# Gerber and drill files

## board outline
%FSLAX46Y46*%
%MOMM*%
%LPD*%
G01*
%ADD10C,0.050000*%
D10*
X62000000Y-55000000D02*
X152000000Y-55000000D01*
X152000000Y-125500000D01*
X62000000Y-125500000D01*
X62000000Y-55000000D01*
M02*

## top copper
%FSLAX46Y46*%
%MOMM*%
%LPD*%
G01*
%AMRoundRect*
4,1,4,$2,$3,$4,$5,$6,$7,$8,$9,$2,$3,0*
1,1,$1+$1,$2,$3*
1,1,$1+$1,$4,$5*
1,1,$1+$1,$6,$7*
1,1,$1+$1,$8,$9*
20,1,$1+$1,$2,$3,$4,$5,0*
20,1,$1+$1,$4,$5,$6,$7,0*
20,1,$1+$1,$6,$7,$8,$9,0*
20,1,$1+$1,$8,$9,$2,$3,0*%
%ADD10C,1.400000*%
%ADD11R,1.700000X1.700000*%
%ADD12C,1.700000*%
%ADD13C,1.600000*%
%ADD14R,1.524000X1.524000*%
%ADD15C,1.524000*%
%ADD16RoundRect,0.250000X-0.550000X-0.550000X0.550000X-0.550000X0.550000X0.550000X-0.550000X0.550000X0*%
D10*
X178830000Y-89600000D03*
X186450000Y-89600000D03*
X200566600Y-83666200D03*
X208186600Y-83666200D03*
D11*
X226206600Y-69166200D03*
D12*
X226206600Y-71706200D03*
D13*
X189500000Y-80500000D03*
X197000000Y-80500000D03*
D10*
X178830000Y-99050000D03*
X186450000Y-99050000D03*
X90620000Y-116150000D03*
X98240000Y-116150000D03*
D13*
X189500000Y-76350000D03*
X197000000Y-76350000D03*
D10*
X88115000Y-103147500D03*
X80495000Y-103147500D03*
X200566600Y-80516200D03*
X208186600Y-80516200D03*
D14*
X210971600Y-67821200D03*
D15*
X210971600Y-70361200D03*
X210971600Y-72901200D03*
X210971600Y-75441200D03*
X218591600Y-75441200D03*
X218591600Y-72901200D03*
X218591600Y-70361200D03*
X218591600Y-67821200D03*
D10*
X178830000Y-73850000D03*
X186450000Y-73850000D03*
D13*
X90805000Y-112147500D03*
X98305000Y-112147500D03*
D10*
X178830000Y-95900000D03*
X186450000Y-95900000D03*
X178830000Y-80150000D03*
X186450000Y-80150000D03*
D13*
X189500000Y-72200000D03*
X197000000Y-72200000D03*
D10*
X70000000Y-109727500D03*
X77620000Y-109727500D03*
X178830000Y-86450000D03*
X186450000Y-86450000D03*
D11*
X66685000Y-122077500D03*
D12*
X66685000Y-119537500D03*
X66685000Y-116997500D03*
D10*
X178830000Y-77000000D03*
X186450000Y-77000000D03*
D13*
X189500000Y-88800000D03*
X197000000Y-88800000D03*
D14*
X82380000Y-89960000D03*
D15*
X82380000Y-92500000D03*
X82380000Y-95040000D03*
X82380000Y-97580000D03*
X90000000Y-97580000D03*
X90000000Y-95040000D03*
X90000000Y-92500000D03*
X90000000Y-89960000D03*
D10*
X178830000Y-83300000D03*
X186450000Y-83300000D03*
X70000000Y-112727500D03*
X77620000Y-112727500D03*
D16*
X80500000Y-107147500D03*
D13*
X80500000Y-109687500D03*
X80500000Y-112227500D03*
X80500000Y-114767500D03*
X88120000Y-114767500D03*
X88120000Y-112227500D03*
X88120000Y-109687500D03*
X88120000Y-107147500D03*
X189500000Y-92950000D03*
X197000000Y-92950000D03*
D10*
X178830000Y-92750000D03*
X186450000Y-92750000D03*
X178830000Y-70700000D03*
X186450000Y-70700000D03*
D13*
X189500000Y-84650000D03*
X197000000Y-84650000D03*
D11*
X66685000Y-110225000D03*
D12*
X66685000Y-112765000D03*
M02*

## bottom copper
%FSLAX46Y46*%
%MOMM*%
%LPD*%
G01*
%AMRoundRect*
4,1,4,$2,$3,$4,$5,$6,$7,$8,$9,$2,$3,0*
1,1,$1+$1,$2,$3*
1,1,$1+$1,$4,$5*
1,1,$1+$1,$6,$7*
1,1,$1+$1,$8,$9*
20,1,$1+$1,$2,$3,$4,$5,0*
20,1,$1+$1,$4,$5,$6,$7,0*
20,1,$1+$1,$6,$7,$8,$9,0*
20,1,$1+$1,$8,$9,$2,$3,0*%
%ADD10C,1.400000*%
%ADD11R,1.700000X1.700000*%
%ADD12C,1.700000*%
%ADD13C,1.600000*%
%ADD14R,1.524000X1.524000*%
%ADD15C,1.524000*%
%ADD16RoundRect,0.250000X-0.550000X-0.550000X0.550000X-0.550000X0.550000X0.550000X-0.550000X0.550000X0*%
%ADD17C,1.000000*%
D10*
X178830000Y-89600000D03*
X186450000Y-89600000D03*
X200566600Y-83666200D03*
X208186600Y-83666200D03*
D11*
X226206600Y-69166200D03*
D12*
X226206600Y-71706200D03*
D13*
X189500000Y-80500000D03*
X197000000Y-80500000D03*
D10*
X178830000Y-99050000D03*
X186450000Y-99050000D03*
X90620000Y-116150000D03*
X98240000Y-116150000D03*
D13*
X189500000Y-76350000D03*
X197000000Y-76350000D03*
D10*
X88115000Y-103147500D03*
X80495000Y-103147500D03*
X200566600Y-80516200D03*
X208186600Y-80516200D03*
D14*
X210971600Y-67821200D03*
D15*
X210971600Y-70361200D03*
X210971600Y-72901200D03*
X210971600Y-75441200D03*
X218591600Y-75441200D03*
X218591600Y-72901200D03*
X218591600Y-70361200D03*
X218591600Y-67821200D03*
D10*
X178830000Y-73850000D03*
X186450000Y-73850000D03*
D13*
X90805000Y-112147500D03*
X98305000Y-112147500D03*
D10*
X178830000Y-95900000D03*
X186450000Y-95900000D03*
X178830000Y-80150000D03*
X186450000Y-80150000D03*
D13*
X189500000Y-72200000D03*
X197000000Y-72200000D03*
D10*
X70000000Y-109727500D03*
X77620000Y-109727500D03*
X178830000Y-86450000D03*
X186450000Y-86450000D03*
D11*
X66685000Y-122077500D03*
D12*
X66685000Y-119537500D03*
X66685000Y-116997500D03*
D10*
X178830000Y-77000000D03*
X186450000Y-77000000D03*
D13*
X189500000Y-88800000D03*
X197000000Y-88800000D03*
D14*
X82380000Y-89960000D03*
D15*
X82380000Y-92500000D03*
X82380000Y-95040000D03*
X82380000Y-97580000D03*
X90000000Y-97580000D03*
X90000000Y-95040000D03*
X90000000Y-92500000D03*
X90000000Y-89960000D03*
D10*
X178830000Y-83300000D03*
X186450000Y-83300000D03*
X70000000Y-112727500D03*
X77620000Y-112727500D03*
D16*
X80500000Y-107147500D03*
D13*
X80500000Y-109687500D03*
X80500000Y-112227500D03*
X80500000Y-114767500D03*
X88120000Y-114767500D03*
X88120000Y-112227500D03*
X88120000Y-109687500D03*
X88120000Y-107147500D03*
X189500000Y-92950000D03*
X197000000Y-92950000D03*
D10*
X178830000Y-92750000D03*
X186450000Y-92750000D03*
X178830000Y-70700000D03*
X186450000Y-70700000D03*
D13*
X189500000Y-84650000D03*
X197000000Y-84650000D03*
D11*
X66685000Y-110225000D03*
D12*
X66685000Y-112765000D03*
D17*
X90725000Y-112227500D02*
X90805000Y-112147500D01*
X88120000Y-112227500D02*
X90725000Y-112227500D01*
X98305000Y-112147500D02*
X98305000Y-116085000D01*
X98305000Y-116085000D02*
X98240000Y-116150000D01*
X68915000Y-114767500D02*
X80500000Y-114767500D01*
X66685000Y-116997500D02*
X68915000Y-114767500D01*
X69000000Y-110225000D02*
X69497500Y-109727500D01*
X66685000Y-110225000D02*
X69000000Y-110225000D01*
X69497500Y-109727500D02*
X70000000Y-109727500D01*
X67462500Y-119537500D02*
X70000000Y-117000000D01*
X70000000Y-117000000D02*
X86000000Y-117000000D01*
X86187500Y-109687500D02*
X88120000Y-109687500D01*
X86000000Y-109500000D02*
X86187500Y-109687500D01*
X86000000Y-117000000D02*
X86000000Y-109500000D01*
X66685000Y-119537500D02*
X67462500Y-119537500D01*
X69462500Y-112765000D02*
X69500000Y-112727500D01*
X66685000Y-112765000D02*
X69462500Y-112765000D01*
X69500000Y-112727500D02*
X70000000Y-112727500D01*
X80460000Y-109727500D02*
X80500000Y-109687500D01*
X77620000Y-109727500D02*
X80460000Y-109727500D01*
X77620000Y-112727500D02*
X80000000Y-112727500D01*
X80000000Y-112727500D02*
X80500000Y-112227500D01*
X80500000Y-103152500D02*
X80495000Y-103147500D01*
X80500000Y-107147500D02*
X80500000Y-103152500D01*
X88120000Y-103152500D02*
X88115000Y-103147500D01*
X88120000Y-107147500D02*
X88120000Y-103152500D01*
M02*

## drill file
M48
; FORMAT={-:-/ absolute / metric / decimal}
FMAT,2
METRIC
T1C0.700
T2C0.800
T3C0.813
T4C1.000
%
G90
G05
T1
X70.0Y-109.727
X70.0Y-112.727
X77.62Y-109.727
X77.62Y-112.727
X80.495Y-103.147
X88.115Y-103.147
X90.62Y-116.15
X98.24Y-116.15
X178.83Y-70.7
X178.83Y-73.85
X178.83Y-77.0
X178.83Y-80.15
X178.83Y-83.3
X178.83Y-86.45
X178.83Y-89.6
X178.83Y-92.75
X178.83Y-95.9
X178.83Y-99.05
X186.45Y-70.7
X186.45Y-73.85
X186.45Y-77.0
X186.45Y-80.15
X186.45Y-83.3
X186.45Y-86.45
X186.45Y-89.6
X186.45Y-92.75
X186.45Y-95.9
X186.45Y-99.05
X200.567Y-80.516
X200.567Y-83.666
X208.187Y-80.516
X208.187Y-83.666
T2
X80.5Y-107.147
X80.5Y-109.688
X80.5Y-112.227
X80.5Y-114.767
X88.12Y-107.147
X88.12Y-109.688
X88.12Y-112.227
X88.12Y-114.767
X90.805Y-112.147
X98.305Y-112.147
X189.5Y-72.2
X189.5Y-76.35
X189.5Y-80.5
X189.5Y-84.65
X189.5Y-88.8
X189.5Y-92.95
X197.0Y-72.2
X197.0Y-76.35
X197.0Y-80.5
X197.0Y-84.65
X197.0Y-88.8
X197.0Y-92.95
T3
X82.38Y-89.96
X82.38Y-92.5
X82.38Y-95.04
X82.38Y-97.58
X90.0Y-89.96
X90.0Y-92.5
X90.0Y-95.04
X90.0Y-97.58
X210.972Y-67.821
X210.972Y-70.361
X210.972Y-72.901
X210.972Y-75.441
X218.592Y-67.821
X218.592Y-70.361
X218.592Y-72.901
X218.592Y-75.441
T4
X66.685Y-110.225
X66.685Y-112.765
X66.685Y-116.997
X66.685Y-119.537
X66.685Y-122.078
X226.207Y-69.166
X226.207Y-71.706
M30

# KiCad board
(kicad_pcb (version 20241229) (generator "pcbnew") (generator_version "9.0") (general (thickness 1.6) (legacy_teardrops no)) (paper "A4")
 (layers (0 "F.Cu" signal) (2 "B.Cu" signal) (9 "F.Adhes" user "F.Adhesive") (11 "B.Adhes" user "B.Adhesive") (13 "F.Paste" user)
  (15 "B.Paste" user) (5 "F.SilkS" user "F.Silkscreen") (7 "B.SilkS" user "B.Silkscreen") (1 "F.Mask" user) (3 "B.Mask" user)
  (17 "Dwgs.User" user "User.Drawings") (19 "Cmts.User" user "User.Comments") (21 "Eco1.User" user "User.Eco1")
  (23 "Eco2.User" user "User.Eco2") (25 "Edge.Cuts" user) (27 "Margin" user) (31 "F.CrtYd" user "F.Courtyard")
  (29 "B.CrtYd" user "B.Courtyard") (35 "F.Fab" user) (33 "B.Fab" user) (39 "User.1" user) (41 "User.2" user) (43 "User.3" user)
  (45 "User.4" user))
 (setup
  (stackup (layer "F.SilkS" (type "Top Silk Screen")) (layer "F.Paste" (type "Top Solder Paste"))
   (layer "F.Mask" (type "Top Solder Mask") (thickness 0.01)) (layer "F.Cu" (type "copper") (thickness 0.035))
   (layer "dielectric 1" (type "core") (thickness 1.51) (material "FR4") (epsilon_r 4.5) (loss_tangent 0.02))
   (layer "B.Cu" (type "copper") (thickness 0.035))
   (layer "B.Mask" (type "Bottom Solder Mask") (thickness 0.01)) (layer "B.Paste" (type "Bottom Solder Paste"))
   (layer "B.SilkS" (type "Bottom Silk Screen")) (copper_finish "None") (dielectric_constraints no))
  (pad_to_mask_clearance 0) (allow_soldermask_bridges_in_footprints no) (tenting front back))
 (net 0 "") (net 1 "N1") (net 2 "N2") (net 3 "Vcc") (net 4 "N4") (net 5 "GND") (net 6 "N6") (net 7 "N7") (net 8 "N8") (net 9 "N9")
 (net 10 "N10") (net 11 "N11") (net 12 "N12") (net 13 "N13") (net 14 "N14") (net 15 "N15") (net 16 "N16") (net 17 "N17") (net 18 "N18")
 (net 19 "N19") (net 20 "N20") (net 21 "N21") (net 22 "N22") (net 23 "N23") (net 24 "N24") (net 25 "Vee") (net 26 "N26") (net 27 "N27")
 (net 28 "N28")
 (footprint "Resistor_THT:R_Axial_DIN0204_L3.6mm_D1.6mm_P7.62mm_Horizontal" (layer "F.Cu") (at 178.83 89.6)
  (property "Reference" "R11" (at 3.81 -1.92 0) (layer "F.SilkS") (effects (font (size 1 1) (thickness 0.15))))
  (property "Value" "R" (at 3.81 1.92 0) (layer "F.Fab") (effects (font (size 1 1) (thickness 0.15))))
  (pad "1" thru_hole circle (at 0 0) (size 1.4 1.4) (drill 0.7) (layers "*.Cu" "*.Mask") (remove_unused_layers no) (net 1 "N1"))
  (pad "2" thru_hole circle (at 7.62 0) (size 1.4 1.4) (drill 0.7) (layers "*.Cu" "*.Mask") (remove_unused_layers no) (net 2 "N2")))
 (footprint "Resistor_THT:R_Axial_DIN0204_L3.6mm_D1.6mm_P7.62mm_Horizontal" (layer "F.Cu") (at 200.5666 83.6662)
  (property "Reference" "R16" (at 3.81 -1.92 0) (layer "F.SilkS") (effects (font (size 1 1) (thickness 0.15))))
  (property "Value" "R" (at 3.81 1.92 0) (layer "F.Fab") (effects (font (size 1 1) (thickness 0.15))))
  (pad "1" thru_hole circle (at 0 0) (size 1.4 1.4) (drill 0.7) (layers "*.Cu" "*.Mask") (remove_unused_layers no) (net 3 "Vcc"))
  (pad "2" thru_hole circle (at 7.62 0) (size 1.4 1.4) (drill 0.7) (layers "*.Cu" "*.Mask") (remove_unused_layers no) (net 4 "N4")))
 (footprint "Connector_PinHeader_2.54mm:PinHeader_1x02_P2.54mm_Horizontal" (layer "F.Cu") (at 226.2066 69.1662)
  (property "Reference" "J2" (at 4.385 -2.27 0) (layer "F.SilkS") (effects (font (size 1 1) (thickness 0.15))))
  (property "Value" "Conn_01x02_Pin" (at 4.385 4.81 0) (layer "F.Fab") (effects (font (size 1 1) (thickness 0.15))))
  (pad "1" thru_hole rect (at 0 0) (size 1.7 1.7) (drill 1) (layers "*.Cu" "*.Mask") (remove_unused_layers no) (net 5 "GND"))
  (pad "2" thru_hole circle (at 0 2.54) (size 1.7 1.7) (drill 1) (layers "*.Cu" "*.Mask") (remove_unused_layers no) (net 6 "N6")))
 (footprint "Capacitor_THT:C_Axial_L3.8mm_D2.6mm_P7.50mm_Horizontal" (layer "F.Cu") (at 189.5 80.5)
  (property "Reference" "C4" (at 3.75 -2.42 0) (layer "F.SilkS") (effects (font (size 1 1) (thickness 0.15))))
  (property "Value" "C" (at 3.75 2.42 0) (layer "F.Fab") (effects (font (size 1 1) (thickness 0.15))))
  (pad "1" thru_hole circle (at 0 0) (size 1.6 1.6) (drill 0.8) (layers "*.Cu" "*.Mask") (remove_unused_layers no) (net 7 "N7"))
  (pad "2" thru_hole circle (at 7.5 0) (size 1.6 1.6) (drill 0.8) (layers "*.Cu" "*.Mask") (remove_unused_layers no) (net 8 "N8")))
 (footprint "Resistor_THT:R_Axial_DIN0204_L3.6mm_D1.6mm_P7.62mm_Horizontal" (layer "F.Cu") (at 178.83 99.05)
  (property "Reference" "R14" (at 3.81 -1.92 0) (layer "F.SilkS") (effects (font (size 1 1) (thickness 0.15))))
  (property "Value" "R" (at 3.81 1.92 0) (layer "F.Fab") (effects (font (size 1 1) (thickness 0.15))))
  (pad "1" thru_hole circle (at 0 0) (size 1.4 1.4) (drill 0.7) (layers "*.Cu" "*.Mask") (remove_unused_layers no) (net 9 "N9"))
  (pad "2" thru_hole circle (at 7.62 0) (size 1.4 1.4) (drill 0.7) (layers "*.Cu" "*.Mask") (remove_unused_layers no) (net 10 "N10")))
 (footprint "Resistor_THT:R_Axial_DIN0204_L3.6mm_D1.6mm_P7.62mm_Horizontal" (layer "F.Cu") (at 90.62 116.15)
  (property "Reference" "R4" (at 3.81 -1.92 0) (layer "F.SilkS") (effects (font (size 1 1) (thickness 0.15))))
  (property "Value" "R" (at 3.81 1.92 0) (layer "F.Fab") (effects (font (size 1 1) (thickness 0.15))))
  (pad "1" thru_hole circle (at 0 0) (size 1.4 1.4) (drill 0.7) (layers "*.Cu" "*.Mask") (remove_unused_layers no) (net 5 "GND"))
  (pad "2" thru_hole circle (at 7.62 0) (size 1.4 1.4) (drill 0.7) (layers "*.Cu" "*.Mask") (remove_unused_layers no) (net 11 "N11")))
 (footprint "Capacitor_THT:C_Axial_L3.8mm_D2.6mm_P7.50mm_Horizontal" (layer "F.Cu") (at 189.5 76.35)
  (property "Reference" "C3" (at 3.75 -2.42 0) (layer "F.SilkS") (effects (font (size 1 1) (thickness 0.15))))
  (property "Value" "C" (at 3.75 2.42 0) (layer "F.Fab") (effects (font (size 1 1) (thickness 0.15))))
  (pad "1" thru_hole circle (at 0 0) (size 1.6 1.6) (drill 0.8) (layers "*.Cu" "*.Mask") (remove_unused_layers no) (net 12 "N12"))
  (pad "2" thru_hole circle (at 7.5 0) (size 1.6 1.6) (drill 0.8) (layers "*.Cu" "*.Mask") (remove_unused_layers no) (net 5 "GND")))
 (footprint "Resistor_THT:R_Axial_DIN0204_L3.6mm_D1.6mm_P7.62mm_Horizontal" (layer "F.Cu") (at 88.115 103.1475 180)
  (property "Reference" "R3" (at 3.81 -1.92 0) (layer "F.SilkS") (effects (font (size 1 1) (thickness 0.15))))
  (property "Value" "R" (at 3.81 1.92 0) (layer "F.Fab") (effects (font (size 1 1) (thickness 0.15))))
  (pad "1" thru_hole circle (at 0 0 180) (size 1.4 1.4) (drill 0.7) (layers "*.Cu" "*.Mask") (remove_unused_layers no) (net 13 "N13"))
  (pad "2" thru_hole circle (at 7.62 0 180) (size 1.4 1.4) (drill 0.7) (layers "*.Cu" "*.Mask") (remove_unused_layers no) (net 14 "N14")))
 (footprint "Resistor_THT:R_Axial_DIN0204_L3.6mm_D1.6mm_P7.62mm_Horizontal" (layer "F.Cu") (at 200.5666 80.5162)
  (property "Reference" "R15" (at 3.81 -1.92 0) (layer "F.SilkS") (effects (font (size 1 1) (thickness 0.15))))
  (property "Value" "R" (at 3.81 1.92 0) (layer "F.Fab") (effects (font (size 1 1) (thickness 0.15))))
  (pad "1" thru_hole circle (at 0 0) (size 1.4 1.4) (drill 0.7) (layers "*.Cu" "*.Mask") (remove_unused_layers no) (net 5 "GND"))
  (pad "2" thru_hole circle (at 7.62 0) (size 1.4 1.4) (drill 0.7) (layers "*.Cu" "*.Mask") (remove_unused_layers no) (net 4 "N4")))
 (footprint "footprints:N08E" (layer "F.Cu") (at 218.5916 75.4412)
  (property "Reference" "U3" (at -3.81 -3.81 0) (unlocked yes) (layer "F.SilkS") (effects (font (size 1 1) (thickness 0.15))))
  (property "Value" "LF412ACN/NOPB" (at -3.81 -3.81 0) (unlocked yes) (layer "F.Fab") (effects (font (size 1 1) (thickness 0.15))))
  (pad "1" thru_hole rect (at -7.62 -7.62) (size 1.524 1.524) (drill 0.8128) (layers "*.Cu" "*.Mask") (remove_unused_layers no)
   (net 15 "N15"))
  (pad "2" thru_hole circle (at -7.62 -5.08) (size 1.524 1.524) (drill 0.8128) (layers "*.Cu" "*.Mask") (remove_unused_layers no)
   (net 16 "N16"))
  (pad "3" thru_hole circle (at -7.62 -2.54) (size 1.524 1.524) (drill 0.8128) (layers "*.Cu" "*.Mask") (remove_unused_layers no)
   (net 5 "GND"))
  (pad "4" thru_hole circle (at -7.62 0) (size 1.524 1.524) (drill 0.8128) (layers "*.Cu" "*.Mask") (remove_unused_layers no))
  (pad "5" thru_hole circle (at 0 0) (size 1.524 1.524) (drill 0.8128) (layers "*.Cu" "*.Mask") (remove_unused_layers no) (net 4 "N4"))
  (pad "6" thru_hole circle (at 0 -2.54) (size 1.524 1.524) (drill 0.8128) (layers "*.Cu" "*.Mask") (remove_unused_layers no) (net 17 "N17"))
  (pad "7" thru_hole circle (at 0 -5.08) (size 1.524 1.524) (drill 0.8128) (layers "*.Cu" "*.Mask") (remove_unused_layers no) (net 6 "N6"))
  (pad "8" thru_hole circle (at 0 -7.62) (size 1.524 1.524) (drill 0.8128) (layers "*.Cu" "*.Mask") (remove_unused_layers no)))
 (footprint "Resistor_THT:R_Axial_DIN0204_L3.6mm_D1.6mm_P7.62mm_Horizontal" (layer "F.Cu") (at 178.83 73.85)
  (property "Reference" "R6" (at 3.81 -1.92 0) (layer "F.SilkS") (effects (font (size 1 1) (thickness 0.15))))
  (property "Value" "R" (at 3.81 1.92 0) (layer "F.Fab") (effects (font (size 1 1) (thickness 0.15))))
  (pad "1" thru_hole circle (at 0 0) (size 1.4 1.4) (drill 0.7) (layers "*.Cu" "*.Mask") (remove_unused_layers no) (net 12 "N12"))
  (pad "2" thru_hole circle (at 7.62 0) (size 1.4 1.4) (drill 0.7) (layers "*.Cu" "*.Mask") (remove_unused_layers no) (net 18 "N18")))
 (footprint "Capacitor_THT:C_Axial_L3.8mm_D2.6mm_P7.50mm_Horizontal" (layer "F.Cu") (at 90.805 112.1475)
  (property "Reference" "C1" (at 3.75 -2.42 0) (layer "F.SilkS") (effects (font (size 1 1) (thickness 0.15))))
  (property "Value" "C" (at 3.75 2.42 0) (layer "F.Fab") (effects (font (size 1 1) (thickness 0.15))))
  (pad "1" thru_hole circle (at 0 0) (size 1.6 1.6) (drill 0.8) (layers "*.Cu" "*.Mask") (remove_unused_layers no) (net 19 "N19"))
  (pad "2" thru_hole circle (at 7.5 0) (size 1.6 1.6) (drill 0.8) (layers "*.Cu" "*.Mask") (remove_unused_layers no) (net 11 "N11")))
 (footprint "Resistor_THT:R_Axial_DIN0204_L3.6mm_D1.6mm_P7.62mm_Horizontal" (layer "F.Cu") (at 178.83 95.9)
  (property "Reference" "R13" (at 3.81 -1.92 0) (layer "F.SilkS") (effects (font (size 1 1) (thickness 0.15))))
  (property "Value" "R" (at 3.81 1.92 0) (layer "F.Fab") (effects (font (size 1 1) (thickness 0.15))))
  (pad "1" thru_hole circle (at 0 0) (size 1.4 1.4) (drill 0.7) (layers "*.Cu" "*.Mask") (remove_unused_layers no) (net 5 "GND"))
  (pad "2" thru_hole circle (at 7.62 0) (size 1.4 1.4) (drill 0.7) (layers "*.Cu" "*.Mask") (remove_unused_layers no) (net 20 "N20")))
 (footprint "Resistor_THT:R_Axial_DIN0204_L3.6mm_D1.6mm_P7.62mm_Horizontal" (layer "F.Cu") (at 178.83 80.15)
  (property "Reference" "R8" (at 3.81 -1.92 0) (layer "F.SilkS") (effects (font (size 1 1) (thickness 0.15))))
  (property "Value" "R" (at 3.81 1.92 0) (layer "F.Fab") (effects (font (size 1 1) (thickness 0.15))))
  (pad "1" thru_hole circle (at 0 0) (size 1.4 1.4) (drill 0.7) (layers "*.Cu" "*.Mask") (remove_unused_layers no) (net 5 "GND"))
  (pad "2" thru_hole circle (at 7.62 0) (size 1.4 1.4) (drill 0.7) (layers "*.Cu" "*.Mask") (remove_unused_layers no) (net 7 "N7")))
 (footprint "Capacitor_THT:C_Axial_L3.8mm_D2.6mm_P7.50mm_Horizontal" (layer "F.Cu") (at 189.5 72.2)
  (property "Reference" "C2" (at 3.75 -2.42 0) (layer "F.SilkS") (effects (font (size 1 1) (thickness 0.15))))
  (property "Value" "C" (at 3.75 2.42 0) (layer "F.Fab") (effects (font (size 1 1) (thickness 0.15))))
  (pad "1" thru_hole circle (at 0 0) (size 1.6 1.6) (drill 0.8) (layers "*.Cu" "*.Mask") (remove_unused_layers no) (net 12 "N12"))
  (pad "2" thru_hole circle (at 7.5 0) (size 1.6 1.6) (drill 0.8) (layers "*.Cu" "*.Mask") (remove_unused_layers no) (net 5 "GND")))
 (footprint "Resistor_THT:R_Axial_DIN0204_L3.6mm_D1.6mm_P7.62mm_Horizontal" (layer "F.Cu") (at 70 109.7275)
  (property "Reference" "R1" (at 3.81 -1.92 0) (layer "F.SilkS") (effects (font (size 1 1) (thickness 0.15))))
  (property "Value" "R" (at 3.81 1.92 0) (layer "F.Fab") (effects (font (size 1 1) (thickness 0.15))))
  (pad "1" thru_hole circle (at 0 0) (size 1.4 1.4) (drill 0.7) (layers "*.Cu" "*.Mask") (remove_unused_layers no) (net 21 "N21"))
  (pad "2" thru_hole circle (at 7.62 0) (size 1.4 1.4) (drill 0.7) (layers "*.Cu" "*.Mask") (remove_unused_layers no) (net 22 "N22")))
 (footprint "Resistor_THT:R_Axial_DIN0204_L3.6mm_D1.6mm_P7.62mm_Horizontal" (layer "F.Cu") (at 178.83 86.45)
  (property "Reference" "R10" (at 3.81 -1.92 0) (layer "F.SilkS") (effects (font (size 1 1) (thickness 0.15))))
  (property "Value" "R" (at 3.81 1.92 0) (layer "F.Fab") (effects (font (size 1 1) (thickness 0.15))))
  (pad "1" thru_hole circle (at 0 0) (size 1.4 1.4) (drill 0.7) (layers "*.Cu" "*.Mask") (remove_unused_layers no) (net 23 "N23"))
  (pad "2" thru_hole circle (at 7.62 0) (size 1.4 1.4) (drill 0.7) (layers "*.Cu" "*.Mask") (remove_unused_layers no) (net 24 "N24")))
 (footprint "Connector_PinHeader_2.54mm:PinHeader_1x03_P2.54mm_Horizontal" (layer "F.Cu") (at 66.685 122.0775 180)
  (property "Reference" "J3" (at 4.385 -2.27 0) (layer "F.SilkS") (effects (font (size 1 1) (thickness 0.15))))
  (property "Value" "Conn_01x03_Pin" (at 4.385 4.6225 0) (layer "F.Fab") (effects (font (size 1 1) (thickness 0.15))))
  (pad "1" thru_hole rect (at 0 0 180) (size 1.7 1.7) (drill 1) (layers "*.Cu" "*.Mask") (remove_unused_layers no) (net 5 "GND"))
  (pad "2" thru_hole circle (at 0 2.54 180) (size 1.7 1.7) (drill 1) (layers "*.Cu" "*.Mask") (remove_unused_layers no) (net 3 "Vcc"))
  (pad "3" thru_hole circle (at 0 5.08 180) (size 1.7 1.7) (drill 1) (layers "*.Cu" "*.Mask") (remove_unused_layers no) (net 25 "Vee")))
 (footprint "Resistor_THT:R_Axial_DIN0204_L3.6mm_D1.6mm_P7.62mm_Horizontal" (layer "F.Cu") (at 178.83 77)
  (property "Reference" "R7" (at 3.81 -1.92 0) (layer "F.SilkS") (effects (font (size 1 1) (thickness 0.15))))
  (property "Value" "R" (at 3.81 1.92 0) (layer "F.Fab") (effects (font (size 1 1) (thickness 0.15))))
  (pad "1" thru_hole circle (at 0 0) (size 1.4 1.4) (drill 0.7) (layers "*.Cu" "*.Mask") (remove_unused_layers no) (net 5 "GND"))
  (pad "2" thru_hole circle (at 7.62 0) (size 1.4 1.4) (drill 0.7) (layers "*.Cu" "*.Mask") (remove_unused_layers no) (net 7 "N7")))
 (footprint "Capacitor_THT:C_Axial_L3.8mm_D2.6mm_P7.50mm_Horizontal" (layer "F.Cu") (at 189.5 88.8)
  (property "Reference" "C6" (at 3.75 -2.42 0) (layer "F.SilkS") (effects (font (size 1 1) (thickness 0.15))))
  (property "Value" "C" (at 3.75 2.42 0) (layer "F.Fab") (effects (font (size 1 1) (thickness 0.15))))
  (pad "1" thru_hole circle (at 0 0) (size 1.6 1.6) (drill 0.8) (layers "*.Cu" "*.Mask") (remove_unused_layers no) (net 23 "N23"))
  (pad "2" thru_hole circle (at 7.5 0) (size 1.6 1.6) (drill 0.8) (layers "*.Cu" "*.Mask") (remove_unused_layers no) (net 24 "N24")))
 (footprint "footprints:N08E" (layer "F.Cu") (at 90 97.58)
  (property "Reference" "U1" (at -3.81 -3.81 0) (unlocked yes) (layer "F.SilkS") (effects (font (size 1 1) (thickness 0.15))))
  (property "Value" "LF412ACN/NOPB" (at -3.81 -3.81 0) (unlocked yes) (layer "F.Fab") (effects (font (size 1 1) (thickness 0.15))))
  (pad "1" thru_hole rect (at -7.62 -7.62) (size 1.524 1.524) (drill 0.8128) (layers "*.Cu" "*.Mask") (remove_unused_layers no) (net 8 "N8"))
  (pad "2" thru_hole circle (at -7.62 -5.08) (size 1.524 1.524) (drill 0.8128) (layers "*.Cu" "*.Mask") (remove_unused_layers no)
   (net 8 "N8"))
  (pad "3" thru_hole circle (at -7.62 -2.54) (size 1.524 1.524) (drill 0.8128) (layers "*.Cu" "*.Mask") (remove_unused_layers no)
   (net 11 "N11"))
  (pad "4" thru_hole circle (at -7.62 0) (size 1.524 1.524) (drill 0.8128) (layers "*.Cu" "*.Mask") (remove_unused_layers no))
  (pad "5" thru_hole circle (at 0 0) (size 1.524 1.524) (drill 0.8128) (layers "*.Cu" "*.Mask") (remove_unused_layers no) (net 18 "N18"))
  (pad "6" thru_hole circle (at 0 -2.54) (size 1.524 1.524) (drill 0.8128) (layers "*.Cu" "*.Mask") (remove_unused_layers no) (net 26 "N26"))
  (pad "7" thru_hole circle (at 0 -5.08) (size 1.524 1.524) (drill 0.8128) (layers "*.Cu" "*.Mask") (remove_unused_layers no) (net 26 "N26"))
  (pad "8" thru_hole circle (at 0 -7.62) (size 1.524 1.524) (drill 0.8128) (layers "*.Cu" "*.Mask") (remove_unused_layers no)))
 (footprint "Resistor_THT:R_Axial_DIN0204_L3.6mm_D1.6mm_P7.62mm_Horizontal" (layer "F.Cu") (at 178.83 83.3)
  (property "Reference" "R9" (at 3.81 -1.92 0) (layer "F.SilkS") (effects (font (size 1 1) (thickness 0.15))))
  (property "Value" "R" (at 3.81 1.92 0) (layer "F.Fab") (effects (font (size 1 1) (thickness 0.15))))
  (pad "1" thru_hole circle (at 0 0) (size 1.4 1.4) (drill 0.7) (layers "*.Cu" "*.Mask") (remove_unused_layers no) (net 26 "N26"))
  (pad "2" thru_hole circle (at 7.62 0) (size 1.4 1.4) (drill 0.7) (layers "*.Cu" "*.Mask") (remove_unused_layers no) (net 16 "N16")))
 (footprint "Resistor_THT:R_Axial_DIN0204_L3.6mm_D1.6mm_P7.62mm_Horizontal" (layer "F.Cu") (at 70 112.7275)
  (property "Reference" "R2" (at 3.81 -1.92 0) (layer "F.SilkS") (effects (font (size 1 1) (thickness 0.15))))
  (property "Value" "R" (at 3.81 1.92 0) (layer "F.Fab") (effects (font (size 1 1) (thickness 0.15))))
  (pad "1" thru_hole circle (at 0 0) (size 1.4 1.4) (drill 0.7) (layers "*.Cu" "*.Mask") (remove_unused_layers no) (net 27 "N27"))
  (pad "2" thru_hole circle (at 7.62 0) (size 1.4 1.4) (drill 0.7) (layers "*.Cu" "*.Mask") (remove_unused_layers no) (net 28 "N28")))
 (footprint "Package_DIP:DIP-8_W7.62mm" (layer "F.Cu") (at 80.5 107.1475)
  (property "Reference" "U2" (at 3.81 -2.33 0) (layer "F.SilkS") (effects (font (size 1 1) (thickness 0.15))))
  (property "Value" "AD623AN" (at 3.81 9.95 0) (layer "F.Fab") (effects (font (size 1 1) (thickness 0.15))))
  (pad "1" thru_hole roundrect (at 0 0) (size 1.6 1.6) (drill 0.8) (layers "*.Cu" "*.Mask") (remove_unused_layers no)
   (roundrect_rratio 0.15625) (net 14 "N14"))
  (pad "2" thru_hole circle (at 0 2.54) (size 1.6 1.6) (drill 0.8) (layers "*.Cu" "*.Mask") (remove_unused_layers no) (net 22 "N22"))
  (pad "3" thru_hole circle (at 0 5.08) (size 1.6 1.6) (drill 0.8) (layers "*.Cu" "*.Mask") (remove_unused_layers no) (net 28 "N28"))
  (pad "4" thru_hole circle (at 0 7.62) (size 1.6 1.6) (drill 0.8) (layers "*.Cu" "*.Mask") (remove_unused_layers no) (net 25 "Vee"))
  (pad "5" thru_hole circle (at 7.62 7.62) (size 1.6 1.6) (drill 0.8) (layers "*.Cu" "*.Mask") (remove_unused_layers no) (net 5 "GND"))
  (pad "6" thru_hole circle (at 7.62 5.08) (size 1.6 1.6) (drill 0.8) (layers "*.Cu" "*.Mask") (remove_unused_layers no) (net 19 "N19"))
  (pad "7" thru_hole circle (at 7.62 2.54) (size 1.6 1.6) (drill 0.8) (layers "*.Cu" "*.Mask") (remove_unused_layers no) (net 3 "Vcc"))
  (pad "8" thru_hole circle (at 7.62 0) (size 1.6 1.6) (drill 0.8) (layers "*.Cu" "*.Mask") (remove_unused_layers no) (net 13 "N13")))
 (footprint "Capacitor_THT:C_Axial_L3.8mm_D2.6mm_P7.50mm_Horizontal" (layer "F.Cu") (at 189.5 92.95)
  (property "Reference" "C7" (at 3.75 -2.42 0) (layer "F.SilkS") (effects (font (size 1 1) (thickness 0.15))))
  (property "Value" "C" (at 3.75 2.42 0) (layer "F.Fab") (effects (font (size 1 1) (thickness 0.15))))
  (pad "1" thru_hole circle (at 0 0) (size 1.6 1.6) (drill 0.8) (layers "*.Cu" "*.Mask") (remove_unused_layers no) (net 15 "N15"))
  (pad "2" thru_hole circle (at 7.5 0) (size 1.6 1.6) (drill 0.8) (layers "*.Cu" "*.Mask") (remove_unused_layers no) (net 1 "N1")))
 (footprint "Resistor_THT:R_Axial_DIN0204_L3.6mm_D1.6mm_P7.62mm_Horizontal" (layer "F.Cu") (at 178.83 92.75)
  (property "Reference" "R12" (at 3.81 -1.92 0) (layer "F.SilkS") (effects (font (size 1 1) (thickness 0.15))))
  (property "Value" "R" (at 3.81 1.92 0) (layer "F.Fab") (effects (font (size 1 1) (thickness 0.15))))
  (pad "1" thru_hole circle (at 0 0) (size 1.4 1.4) (drill 0.7) (layers "*.Cu" "*.Mask") (remove_unused_layers no) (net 2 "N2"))
  (pad "2" thru_hole circle (at 7.62 0) (size 1.4 1.4) (drill 0.7) (layers "*.Cu" "*.Mask") (remove_unused_layers no) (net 17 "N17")))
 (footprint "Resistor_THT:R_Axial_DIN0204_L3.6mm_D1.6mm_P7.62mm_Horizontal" (layer "F.Cu") (at 178.83 70.7)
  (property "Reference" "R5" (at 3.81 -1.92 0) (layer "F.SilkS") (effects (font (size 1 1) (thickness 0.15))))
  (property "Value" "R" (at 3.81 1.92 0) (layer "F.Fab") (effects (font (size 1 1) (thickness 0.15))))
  (pad "1" thru_hole circle (at 0 0) (size 1.4 1.4) (drill 0.7) (layers "*.Cu" "*.Mask") (remove_unused_layers no) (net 8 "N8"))
  (pad "2" thru_hole circle (at 7.62 0) (size 1.4 1.4) (drill 0.7) (layers "*.Cu" "*.Mask") (remove_unused_layers no) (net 12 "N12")))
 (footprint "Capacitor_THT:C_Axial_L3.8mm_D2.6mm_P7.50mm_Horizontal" (layer "F.Cu") (at 189.5 84.65)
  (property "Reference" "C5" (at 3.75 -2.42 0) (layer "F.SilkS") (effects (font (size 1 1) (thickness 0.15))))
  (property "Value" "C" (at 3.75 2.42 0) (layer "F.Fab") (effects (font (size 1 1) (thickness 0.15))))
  (pad "1" thru_hole circle (at 0 0) (size 1.6 1.6) (drill 0.8) (layers "*.Cu" "*.Mask") (remove_unused_layers no) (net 18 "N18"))
  (pad "2" thru_hole circle (at 7.5 0) (size 1.6 1.6) (drill 0.8) (layers "*.Cu" "*.Mask") (remove_unused_layers no) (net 7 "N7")))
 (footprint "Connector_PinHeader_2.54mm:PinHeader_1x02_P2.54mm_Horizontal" (layer "B.Cu") (at 66.685 110.225 180)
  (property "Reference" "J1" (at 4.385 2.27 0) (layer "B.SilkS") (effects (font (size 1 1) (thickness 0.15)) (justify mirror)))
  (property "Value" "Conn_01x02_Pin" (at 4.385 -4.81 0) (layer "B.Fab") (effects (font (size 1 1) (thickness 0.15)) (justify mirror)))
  (pad "1" thru_hole rect (at 0 0 180) (size 1.7 1.7) (drill 1) (layers "*.Cu" "*.Mask") (remove_unused_layers no) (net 21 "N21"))
  (pad "2" thru_hole circle (at 0 -2.54 180) (size 1.7 1.7) (drill 1) (layers "*.Cu" "*.Mask") (remove_unused_layers no) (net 27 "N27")))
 (gr_rect (start 62 55) (end 152 125.5) (stroke (width 0.05) (type default)) (fill no) (layer "Edge.Cuts"))
 (segment (start 90.725 112.2275) (end 90.805 112.1475) (width 1) (layer "B.Cu") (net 19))
 (segment (start 88.12 112.2275) (end 90.725 112.2275) (width 1) (layer "B.Cu") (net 19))
 (segment (start 98.305 112.1475) (end 98.305 116.085) (width 1) (layer "B.Cu") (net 11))
 (segment (start 98.305 116.085) (end 98.24 116.15) (width 1) (layer "B.Cu") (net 11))
 (segment (start 68.915 114.7675) (end 80.5 114.7675) (width 1) (layer "B.Cu") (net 25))
 (segment (start 66.685 116.9975) (end 68.915 114.7675) (width 1) (layer "B.Cu") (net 25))
 (segment (start 69 110.225) (end 69.4975 109.7275) (width 1) (layer "B.Cu") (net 21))
 (segment (start 66.685 110.225) (end 69 110.225) (width 1) (layer "B.Cu") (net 21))
 (segment (start 69.4975 109.7275) (end 70 109.7275) (width 1) (layer "B.Cu") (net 21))
 (segment (start 67.4625 119.5375) (end 70 117) (width 1) (layer "B.Cu") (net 3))
 (segment (start 70 117) (end 86 117) (width 1) (layer "B.Cu") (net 3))
 (segment (start 86.1875 109.6875) (end 88.12 109.6875) (width 1) (layer "B.Cu") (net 3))
 (segment (start 86 109.5) (end 86.1875 109.6875) (width 1) (layer "B.Cu") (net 3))
 (segment (start 86 117) (end 86 109.5) (width 1) (layer "B.Cu") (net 3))
 (segment (start 66.685 119.5375) (end 67.4625 119.5375) (width 1) (layer "B.Cu") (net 3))
 (segment (start 69.4625 112.765) (end 69.5 112.7275) (width 1) (layer "B.Cu") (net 27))
 (segment (start 66.685 112.765) (end 69.4625 112.765) (width 1) (layer "B.Cu") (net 27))
 (segment (start 69.5 112.7275) (end 70 112.7275) (width 1) (layer "B.Cu") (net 27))
 (segment (start 80.46 109.7275) (end 80.5 109.6875) (width 1) (layer "B.Cu") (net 22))
 (segment (start 77.62 109.7275) (end 80.46 109.7275) (width 1) (layer "B.Cu") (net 22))
 (segment (start 77.62 112.7275) (end 80 112.7275) (width 1) (layer "B.Cu") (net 28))
 (segment (start 80 112.7275) (end 80.5 112.2275) (width 1) (layer "B.Cu") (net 28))
 (segment (start 80.5 103.1525) (end 80.495 103.1475) (width 1) (layer "B.Cu") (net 14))
 (segment (start 80.5 107.1475) (end 80.5 103.1525) (width 1) (layer "B.Cu") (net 14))
 (segment (start 88.12 103.1525) (end 88.115 103.1475) (width 1) (layer "B.Cu") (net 13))
 (segment (start 88.12 107.1475) (end 88.12 103.1525) (width 1) (layer "B.Cu") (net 13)))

